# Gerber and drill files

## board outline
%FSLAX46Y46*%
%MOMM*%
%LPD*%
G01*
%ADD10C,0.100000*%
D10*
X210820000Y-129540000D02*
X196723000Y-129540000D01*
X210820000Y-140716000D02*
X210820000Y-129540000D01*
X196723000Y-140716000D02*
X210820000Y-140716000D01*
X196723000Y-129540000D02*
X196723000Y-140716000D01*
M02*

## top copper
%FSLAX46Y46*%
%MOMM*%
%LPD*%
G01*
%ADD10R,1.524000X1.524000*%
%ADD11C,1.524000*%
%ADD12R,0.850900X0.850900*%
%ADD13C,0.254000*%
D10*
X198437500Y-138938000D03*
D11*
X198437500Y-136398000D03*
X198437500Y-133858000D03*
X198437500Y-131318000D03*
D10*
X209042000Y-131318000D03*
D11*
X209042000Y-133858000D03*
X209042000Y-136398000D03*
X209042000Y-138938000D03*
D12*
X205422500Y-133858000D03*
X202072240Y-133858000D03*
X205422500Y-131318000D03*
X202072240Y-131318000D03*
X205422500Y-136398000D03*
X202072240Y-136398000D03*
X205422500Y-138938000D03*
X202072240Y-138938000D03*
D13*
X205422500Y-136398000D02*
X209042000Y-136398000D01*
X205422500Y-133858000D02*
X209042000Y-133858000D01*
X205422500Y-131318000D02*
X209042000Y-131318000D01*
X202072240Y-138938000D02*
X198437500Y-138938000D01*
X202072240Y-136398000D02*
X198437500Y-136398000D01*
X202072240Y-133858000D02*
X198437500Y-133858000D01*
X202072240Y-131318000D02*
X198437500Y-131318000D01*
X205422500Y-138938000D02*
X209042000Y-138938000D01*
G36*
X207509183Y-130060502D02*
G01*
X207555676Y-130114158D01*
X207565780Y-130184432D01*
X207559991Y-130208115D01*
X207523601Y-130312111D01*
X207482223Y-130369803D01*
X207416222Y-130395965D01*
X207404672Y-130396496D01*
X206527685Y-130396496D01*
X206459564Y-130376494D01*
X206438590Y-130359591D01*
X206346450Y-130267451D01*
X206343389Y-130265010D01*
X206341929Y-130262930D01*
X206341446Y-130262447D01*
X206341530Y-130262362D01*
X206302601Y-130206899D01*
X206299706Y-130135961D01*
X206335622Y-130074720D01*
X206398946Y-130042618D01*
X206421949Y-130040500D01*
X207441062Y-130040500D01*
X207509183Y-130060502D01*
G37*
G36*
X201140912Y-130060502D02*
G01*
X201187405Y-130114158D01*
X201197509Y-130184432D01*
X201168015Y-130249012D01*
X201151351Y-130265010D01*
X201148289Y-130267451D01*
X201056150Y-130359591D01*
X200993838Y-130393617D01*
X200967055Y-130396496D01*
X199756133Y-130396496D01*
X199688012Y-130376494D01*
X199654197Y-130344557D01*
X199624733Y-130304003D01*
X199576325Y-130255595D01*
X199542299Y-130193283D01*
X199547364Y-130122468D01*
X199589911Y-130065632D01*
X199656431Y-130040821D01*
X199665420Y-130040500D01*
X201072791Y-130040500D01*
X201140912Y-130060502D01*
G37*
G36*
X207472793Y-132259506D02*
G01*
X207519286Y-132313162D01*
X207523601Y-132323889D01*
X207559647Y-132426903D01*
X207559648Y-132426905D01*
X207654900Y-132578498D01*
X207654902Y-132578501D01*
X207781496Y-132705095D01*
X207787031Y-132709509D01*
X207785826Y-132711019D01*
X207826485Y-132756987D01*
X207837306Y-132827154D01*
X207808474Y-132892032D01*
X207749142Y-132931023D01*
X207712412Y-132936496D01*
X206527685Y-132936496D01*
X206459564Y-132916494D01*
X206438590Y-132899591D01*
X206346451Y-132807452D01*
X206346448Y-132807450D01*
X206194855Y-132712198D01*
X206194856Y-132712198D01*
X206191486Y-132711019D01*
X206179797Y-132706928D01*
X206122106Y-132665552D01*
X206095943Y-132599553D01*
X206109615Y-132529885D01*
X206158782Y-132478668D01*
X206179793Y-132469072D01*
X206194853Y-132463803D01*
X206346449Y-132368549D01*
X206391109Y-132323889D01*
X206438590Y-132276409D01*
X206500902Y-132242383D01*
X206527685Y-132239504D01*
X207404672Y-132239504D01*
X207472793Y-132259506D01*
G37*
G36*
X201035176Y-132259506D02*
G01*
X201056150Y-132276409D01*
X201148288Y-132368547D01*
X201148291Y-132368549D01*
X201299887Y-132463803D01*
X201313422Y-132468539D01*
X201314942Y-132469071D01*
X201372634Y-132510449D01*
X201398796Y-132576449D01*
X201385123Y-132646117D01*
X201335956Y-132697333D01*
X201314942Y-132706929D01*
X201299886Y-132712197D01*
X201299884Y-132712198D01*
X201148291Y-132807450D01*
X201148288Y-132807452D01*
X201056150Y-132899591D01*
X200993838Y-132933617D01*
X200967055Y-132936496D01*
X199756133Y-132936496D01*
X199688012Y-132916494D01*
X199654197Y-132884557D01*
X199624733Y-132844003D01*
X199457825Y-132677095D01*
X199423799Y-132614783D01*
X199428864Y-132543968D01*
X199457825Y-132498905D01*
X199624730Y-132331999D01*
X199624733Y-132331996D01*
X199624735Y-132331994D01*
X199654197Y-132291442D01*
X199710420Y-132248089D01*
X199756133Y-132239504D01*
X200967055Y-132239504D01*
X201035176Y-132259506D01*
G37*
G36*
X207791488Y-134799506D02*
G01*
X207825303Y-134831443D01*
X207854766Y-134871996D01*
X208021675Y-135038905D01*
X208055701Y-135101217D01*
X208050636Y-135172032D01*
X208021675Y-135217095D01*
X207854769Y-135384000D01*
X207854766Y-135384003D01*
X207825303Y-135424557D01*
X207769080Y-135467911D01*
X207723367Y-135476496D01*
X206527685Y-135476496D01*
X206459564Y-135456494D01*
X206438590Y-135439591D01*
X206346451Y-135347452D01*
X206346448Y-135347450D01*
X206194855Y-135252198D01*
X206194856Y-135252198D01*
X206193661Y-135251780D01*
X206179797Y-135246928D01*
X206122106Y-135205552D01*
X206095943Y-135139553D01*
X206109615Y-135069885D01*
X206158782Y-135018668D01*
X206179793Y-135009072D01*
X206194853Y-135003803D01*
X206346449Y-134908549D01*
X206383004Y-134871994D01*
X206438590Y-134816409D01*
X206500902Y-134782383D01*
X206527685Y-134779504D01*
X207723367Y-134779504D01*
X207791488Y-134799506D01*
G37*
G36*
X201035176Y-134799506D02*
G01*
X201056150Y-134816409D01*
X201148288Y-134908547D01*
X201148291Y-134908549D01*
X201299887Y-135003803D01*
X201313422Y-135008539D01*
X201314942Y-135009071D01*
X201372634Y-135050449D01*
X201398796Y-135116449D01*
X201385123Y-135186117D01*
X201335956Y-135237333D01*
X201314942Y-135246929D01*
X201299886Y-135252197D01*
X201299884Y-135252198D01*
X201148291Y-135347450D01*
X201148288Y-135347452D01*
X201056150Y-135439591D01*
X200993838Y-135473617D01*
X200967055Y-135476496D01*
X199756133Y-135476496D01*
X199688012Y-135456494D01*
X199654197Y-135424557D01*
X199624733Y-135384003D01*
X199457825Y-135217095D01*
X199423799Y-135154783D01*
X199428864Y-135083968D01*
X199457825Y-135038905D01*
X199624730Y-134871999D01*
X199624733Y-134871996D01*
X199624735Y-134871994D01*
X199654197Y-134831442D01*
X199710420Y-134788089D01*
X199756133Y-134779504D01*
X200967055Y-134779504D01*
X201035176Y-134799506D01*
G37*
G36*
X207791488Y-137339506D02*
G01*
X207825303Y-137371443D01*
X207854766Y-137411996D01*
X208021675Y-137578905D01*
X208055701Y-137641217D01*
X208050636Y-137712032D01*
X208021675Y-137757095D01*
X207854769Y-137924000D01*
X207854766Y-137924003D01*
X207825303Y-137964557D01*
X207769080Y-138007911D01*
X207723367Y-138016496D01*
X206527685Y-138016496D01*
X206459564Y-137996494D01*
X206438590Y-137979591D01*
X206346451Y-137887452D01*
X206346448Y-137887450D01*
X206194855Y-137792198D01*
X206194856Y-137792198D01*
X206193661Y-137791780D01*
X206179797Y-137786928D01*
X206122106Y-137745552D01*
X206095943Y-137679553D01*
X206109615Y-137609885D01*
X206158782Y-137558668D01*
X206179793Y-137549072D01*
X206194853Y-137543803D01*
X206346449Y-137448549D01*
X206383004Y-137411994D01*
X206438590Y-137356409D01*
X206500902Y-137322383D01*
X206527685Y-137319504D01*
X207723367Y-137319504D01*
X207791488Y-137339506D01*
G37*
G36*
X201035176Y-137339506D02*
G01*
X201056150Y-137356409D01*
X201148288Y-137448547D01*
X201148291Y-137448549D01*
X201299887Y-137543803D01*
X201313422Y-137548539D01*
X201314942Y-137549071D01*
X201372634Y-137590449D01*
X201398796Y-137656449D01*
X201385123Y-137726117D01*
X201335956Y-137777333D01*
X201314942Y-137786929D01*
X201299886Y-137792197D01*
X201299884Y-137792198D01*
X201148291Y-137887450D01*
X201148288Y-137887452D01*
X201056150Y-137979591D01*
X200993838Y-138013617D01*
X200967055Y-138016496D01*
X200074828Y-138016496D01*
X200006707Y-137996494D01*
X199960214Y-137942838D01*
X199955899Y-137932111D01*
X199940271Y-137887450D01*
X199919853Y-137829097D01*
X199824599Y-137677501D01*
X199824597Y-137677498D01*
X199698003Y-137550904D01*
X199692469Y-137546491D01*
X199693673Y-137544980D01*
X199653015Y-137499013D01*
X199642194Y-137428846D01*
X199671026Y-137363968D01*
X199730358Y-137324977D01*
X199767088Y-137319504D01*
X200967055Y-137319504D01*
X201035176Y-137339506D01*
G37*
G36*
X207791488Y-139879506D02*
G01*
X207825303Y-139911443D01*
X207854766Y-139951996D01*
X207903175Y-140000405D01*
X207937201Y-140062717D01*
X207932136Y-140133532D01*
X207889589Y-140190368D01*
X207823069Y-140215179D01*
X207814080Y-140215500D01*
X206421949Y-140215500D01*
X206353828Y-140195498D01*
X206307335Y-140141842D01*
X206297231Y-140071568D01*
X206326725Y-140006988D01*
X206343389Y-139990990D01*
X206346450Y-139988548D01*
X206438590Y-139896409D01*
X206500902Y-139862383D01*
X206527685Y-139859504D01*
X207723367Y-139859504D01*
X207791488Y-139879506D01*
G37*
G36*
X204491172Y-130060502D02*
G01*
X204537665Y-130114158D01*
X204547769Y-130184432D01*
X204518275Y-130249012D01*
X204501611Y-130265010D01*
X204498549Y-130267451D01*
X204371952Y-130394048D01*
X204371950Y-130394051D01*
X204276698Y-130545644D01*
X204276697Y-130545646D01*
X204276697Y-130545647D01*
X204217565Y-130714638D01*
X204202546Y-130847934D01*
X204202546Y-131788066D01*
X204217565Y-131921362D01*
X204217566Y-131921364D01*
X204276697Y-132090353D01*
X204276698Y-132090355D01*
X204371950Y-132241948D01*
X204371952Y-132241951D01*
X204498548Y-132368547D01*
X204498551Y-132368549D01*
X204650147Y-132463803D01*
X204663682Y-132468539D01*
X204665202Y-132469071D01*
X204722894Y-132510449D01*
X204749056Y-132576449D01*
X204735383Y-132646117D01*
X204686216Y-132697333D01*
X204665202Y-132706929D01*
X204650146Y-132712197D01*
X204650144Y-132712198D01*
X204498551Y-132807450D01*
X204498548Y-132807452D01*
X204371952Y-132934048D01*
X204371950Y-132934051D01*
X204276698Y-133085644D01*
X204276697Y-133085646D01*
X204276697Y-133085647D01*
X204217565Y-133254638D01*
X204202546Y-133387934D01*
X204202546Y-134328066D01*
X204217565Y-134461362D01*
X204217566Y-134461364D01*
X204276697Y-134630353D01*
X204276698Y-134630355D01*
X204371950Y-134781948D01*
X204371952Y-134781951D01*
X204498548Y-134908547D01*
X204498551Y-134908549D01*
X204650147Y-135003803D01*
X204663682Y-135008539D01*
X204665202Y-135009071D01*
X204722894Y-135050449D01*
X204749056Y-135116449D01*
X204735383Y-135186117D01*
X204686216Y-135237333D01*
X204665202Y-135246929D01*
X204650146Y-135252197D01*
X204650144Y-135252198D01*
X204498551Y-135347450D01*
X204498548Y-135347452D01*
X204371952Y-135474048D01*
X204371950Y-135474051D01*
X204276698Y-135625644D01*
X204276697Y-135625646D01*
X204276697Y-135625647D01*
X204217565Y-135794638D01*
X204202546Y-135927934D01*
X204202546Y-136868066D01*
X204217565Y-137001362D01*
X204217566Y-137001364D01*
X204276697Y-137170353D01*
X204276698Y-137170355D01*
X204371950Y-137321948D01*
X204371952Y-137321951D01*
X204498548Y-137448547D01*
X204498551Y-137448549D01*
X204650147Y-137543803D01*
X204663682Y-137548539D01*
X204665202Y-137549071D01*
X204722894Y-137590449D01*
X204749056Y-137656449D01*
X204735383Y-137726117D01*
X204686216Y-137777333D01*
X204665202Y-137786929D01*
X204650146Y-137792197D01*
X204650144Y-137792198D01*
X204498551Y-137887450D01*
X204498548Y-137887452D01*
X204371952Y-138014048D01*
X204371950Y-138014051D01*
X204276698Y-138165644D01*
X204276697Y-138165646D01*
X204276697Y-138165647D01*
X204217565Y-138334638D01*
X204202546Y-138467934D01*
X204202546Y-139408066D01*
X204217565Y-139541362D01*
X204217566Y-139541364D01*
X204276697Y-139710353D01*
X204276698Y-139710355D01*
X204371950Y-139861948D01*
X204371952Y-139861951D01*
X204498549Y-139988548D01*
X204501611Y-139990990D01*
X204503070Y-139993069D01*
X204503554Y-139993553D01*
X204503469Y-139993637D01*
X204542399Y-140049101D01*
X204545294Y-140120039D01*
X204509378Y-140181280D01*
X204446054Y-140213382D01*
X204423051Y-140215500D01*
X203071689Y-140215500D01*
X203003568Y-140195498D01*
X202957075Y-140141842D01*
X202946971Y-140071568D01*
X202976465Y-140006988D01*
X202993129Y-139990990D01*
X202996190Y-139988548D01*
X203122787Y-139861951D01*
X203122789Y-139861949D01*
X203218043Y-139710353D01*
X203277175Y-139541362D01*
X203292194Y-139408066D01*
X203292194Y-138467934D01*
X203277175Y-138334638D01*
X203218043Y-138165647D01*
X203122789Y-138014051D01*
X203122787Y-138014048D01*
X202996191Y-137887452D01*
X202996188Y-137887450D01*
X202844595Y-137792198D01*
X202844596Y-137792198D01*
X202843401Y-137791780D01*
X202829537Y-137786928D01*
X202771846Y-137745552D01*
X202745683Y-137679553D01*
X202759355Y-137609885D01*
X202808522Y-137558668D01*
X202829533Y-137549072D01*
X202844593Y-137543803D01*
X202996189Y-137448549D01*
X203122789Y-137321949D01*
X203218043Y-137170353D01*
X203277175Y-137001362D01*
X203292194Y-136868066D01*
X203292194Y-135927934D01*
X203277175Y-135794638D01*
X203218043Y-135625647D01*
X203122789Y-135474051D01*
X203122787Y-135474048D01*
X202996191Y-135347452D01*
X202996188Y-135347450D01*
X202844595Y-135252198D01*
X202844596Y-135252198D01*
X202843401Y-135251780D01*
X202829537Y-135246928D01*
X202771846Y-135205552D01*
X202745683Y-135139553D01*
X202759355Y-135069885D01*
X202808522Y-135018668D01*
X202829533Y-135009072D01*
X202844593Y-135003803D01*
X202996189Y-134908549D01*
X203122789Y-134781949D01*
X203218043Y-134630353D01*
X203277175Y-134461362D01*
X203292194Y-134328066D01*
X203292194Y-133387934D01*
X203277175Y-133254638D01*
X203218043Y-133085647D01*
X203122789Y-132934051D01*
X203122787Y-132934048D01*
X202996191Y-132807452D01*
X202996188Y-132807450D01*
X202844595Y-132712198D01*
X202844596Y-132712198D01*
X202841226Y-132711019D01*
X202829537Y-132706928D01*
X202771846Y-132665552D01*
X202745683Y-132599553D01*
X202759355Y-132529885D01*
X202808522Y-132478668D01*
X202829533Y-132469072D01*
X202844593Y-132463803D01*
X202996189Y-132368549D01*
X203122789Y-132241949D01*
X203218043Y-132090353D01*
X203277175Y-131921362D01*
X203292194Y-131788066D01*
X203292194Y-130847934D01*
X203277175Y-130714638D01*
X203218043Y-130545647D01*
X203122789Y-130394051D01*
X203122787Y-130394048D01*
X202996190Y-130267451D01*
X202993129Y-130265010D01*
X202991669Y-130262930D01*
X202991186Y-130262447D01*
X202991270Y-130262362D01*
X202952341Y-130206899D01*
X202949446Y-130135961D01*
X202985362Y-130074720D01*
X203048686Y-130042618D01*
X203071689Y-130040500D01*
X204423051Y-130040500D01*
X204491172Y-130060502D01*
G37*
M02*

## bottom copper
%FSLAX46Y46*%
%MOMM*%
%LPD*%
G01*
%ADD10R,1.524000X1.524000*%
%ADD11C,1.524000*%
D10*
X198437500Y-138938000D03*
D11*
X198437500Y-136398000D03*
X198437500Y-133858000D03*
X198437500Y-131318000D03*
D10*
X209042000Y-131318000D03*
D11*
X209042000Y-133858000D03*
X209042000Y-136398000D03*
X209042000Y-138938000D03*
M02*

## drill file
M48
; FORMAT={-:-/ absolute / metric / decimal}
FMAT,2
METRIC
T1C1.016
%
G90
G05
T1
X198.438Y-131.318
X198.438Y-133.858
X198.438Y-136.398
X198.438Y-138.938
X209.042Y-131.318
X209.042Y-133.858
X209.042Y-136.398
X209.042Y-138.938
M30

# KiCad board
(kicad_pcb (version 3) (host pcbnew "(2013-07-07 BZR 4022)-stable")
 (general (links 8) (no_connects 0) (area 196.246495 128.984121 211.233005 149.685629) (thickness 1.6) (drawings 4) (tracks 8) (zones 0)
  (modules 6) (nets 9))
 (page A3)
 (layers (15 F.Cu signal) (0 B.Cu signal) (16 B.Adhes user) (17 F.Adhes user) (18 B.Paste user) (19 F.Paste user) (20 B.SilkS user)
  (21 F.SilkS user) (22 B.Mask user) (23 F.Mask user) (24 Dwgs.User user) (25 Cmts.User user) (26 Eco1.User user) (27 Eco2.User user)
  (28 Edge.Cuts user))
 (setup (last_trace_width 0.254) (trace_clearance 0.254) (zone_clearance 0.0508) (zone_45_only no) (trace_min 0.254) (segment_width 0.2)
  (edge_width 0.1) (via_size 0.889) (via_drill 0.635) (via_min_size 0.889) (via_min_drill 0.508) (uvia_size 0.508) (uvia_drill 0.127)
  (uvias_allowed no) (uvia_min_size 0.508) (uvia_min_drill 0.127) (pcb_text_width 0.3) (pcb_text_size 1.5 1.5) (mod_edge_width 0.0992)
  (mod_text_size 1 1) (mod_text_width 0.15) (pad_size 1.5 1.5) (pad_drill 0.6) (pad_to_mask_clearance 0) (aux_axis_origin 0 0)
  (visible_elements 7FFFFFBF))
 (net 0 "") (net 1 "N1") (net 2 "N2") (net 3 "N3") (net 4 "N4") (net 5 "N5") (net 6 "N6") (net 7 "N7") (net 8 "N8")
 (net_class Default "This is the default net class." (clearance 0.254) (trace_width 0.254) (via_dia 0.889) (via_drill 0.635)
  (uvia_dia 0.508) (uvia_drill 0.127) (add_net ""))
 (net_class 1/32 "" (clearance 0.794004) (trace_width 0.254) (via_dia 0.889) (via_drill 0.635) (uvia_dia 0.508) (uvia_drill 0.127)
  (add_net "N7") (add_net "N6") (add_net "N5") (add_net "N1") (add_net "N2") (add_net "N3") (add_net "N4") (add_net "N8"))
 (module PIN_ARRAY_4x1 (layer F.Cu) (at 198.4375 135.128 90)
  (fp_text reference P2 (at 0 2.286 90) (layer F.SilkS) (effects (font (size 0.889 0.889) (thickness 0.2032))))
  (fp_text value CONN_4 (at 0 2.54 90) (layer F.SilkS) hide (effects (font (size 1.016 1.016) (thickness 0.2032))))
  (pad 1 thru_hole rect (at -3.81 0 90) (size 1.524 1.524) (drill 1.016) (layers *.Cu *.Mask F.SilkS) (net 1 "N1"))
  (pad 2 thru_hole circle (at -1.27 0 90) (size 1.524 1.524) (drill 1.016) (layers *.Cu *.Mask F.SilkS) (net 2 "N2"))
  (pad 3 thru_hole circle (at 1.27 0 90) (size 1.524 1.524) (drill 1.016) (layers *.Cu *.Mask F.SilkS) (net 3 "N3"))
  (pad 4 thru_hole circle (at 3.81 0 90) (size 1.524 1.524) (drill 1.016) (layers *.Cu *.Mask F.SilkS) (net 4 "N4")))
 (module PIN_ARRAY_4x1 (layer F.Cu) (at 209.042 135.128 270)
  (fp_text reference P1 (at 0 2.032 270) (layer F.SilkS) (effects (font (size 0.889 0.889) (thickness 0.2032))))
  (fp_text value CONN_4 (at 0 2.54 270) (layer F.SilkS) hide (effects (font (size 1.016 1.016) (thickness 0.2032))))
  (pad 1 thru_hole rect (at -3.81 0 270) (size 1.524 1.524) (drill 1.016) (layers *.Cu *.Mask F.SilkS) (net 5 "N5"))
  (pad 2 thru_hole circle (at -1.27 0 270) (size 1.524 1.524) (drill 1.016) (layers *.Cu *.Mask F.SilkS) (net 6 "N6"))
  (pad 3 thru_hole circle (at 1.27 0 270) (size 1.524 1.524) (drill 1.016) (layers *.Cu *.Mask F.SilkS) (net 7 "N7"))
  (pad 4 thru_hole circle (at 3.81 0 270) (size 1.524 1.524) (drill 1.016) (layers *.Cu *.Mask F.SilkS) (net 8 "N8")))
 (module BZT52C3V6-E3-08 (layer F.Cu) (at 203.708 133.858 180)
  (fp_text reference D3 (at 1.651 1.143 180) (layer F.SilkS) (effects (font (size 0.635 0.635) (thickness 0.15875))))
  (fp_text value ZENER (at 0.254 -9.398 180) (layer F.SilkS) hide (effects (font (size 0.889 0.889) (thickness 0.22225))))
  (pad 1 smd rect (at -1.7145 0 180) (size 0.8509 0.8509) (layers F.Cu F.Paste F.Mask) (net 6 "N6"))
  (pad 2 smd rect (at 1.63576 0 180) (size 0.8509 0.8509) (layers F.Cu F.Paste F.Mask) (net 3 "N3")))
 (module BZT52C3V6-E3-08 (layer F.Cu) (at 203.708 131.318 180)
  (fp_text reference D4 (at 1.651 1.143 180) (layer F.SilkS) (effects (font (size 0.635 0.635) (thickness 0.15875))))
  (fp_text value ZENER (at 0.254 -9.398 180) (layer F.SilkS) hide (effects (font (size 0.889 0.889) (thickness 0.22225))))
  (pad 1 smd rect (at -1.7145 0 180) (size 0.8509 0.8509) (layers F.Cu F.Paste F.Mask) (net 5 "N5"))
  (pad 2 smd rect (at 1.63576 0 180) (size 0.8509 0.8509) (layers F.Cu F.Paste F.Mask) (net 4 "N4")))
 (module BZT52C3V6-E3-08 (layer F.Cu) (at 203.708 136.398 180)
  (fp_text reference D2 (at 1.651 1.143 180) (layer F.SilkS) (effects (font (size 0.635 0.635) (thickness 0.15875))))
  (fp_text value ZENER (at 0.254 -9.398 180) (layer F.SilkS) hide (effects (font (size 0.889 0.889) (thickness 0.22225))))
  (pad 1 smd rect (at -1.7145 0 180) (size 0.8509 0.8509) (layers F.Cu F.Paste F.Mask) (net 7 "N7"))
  (pad 2 smd rect (at 1.63576 0 180) (size 0.8509 0.8509) (layers F.Cu F.Paste F.Mask) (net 2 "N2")))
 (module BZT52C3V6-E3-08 (layer F.Cu) (at 203.708 138.938 180)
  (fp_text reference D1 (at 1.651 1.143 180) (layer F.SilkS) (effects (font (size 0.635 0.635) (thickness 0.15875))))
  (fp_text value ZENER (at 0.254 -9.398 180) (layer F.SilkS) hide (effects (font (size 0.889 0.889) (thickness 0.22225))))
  (pad 1 smd rect (at -1.7145 0 180) (size 0.8509 0.8509) (layers F.Cu F.Paste F.Mask) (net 8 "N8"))
  (pad 2 smd rect (at 1.63576 0 180) (size 0.8509 0.8509) (layers F.Cu F.Paste F.Mask) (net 1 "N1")))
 (gr_line (start 210.82 129.54) (end 196.723 129.54) (angle 90) (layer Edge.Cuts) (width 0.1))
 (gr_line (start 210.82 140.716) (end 210.82 129.54) (angle 90) (layer Edge.Cuts) (width 0.1))
 (gr_line (start 196.723 140.716) (end 210.82 140.716) (angle 90) (layer Edge.Cuts) (width 0.1))
 (gr_line (start 196.723 129.54) (end 196.723 140.716) (angle 90) (layer Edge.Cuts) (width 0.1))
 (segment (start 205.4225 136.398) (end 209.042 136.398) (width 0.254) (layer F.Cu) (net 7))
 (segment (start 205.4225 133.858) (end 209.042 133.858) (width 0.254) (layer F.Cu) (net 6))
 (segment (start 205.4225 131.318) (end 209.042 131.318) (width 0.254) (layer F.Cu) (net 5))
 (segment (start 202.07224 138.938) (end 198.4375 138.938) (width 0.254) (layer F.Cu) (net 1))
 (segment (start 202.07224 136.398) (end 198.4375 136.398) (width 0.254) (layer F.Cu) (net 2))
 (segment (start 202.07224 133.858) (end 198.4375 133.858) (width 0.254) (layer F.Cu) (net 3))
 (segment (start 202.07224 131.318) (end 198.4375 131.318) (width 0.254) (layer F.Cu) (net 4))
 (segment (start 205.4225 138.938) (end 209.042 138.938) (width 0.254) (layer F.Cu) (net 8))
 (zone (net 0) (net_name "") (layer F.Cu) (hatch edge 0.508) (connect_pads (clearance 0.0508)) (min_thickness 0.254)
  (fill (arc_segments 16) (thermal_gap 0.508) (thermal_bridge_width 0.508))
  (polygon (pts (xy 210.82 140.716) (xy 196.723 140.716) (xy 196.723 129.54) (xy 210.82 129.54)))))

